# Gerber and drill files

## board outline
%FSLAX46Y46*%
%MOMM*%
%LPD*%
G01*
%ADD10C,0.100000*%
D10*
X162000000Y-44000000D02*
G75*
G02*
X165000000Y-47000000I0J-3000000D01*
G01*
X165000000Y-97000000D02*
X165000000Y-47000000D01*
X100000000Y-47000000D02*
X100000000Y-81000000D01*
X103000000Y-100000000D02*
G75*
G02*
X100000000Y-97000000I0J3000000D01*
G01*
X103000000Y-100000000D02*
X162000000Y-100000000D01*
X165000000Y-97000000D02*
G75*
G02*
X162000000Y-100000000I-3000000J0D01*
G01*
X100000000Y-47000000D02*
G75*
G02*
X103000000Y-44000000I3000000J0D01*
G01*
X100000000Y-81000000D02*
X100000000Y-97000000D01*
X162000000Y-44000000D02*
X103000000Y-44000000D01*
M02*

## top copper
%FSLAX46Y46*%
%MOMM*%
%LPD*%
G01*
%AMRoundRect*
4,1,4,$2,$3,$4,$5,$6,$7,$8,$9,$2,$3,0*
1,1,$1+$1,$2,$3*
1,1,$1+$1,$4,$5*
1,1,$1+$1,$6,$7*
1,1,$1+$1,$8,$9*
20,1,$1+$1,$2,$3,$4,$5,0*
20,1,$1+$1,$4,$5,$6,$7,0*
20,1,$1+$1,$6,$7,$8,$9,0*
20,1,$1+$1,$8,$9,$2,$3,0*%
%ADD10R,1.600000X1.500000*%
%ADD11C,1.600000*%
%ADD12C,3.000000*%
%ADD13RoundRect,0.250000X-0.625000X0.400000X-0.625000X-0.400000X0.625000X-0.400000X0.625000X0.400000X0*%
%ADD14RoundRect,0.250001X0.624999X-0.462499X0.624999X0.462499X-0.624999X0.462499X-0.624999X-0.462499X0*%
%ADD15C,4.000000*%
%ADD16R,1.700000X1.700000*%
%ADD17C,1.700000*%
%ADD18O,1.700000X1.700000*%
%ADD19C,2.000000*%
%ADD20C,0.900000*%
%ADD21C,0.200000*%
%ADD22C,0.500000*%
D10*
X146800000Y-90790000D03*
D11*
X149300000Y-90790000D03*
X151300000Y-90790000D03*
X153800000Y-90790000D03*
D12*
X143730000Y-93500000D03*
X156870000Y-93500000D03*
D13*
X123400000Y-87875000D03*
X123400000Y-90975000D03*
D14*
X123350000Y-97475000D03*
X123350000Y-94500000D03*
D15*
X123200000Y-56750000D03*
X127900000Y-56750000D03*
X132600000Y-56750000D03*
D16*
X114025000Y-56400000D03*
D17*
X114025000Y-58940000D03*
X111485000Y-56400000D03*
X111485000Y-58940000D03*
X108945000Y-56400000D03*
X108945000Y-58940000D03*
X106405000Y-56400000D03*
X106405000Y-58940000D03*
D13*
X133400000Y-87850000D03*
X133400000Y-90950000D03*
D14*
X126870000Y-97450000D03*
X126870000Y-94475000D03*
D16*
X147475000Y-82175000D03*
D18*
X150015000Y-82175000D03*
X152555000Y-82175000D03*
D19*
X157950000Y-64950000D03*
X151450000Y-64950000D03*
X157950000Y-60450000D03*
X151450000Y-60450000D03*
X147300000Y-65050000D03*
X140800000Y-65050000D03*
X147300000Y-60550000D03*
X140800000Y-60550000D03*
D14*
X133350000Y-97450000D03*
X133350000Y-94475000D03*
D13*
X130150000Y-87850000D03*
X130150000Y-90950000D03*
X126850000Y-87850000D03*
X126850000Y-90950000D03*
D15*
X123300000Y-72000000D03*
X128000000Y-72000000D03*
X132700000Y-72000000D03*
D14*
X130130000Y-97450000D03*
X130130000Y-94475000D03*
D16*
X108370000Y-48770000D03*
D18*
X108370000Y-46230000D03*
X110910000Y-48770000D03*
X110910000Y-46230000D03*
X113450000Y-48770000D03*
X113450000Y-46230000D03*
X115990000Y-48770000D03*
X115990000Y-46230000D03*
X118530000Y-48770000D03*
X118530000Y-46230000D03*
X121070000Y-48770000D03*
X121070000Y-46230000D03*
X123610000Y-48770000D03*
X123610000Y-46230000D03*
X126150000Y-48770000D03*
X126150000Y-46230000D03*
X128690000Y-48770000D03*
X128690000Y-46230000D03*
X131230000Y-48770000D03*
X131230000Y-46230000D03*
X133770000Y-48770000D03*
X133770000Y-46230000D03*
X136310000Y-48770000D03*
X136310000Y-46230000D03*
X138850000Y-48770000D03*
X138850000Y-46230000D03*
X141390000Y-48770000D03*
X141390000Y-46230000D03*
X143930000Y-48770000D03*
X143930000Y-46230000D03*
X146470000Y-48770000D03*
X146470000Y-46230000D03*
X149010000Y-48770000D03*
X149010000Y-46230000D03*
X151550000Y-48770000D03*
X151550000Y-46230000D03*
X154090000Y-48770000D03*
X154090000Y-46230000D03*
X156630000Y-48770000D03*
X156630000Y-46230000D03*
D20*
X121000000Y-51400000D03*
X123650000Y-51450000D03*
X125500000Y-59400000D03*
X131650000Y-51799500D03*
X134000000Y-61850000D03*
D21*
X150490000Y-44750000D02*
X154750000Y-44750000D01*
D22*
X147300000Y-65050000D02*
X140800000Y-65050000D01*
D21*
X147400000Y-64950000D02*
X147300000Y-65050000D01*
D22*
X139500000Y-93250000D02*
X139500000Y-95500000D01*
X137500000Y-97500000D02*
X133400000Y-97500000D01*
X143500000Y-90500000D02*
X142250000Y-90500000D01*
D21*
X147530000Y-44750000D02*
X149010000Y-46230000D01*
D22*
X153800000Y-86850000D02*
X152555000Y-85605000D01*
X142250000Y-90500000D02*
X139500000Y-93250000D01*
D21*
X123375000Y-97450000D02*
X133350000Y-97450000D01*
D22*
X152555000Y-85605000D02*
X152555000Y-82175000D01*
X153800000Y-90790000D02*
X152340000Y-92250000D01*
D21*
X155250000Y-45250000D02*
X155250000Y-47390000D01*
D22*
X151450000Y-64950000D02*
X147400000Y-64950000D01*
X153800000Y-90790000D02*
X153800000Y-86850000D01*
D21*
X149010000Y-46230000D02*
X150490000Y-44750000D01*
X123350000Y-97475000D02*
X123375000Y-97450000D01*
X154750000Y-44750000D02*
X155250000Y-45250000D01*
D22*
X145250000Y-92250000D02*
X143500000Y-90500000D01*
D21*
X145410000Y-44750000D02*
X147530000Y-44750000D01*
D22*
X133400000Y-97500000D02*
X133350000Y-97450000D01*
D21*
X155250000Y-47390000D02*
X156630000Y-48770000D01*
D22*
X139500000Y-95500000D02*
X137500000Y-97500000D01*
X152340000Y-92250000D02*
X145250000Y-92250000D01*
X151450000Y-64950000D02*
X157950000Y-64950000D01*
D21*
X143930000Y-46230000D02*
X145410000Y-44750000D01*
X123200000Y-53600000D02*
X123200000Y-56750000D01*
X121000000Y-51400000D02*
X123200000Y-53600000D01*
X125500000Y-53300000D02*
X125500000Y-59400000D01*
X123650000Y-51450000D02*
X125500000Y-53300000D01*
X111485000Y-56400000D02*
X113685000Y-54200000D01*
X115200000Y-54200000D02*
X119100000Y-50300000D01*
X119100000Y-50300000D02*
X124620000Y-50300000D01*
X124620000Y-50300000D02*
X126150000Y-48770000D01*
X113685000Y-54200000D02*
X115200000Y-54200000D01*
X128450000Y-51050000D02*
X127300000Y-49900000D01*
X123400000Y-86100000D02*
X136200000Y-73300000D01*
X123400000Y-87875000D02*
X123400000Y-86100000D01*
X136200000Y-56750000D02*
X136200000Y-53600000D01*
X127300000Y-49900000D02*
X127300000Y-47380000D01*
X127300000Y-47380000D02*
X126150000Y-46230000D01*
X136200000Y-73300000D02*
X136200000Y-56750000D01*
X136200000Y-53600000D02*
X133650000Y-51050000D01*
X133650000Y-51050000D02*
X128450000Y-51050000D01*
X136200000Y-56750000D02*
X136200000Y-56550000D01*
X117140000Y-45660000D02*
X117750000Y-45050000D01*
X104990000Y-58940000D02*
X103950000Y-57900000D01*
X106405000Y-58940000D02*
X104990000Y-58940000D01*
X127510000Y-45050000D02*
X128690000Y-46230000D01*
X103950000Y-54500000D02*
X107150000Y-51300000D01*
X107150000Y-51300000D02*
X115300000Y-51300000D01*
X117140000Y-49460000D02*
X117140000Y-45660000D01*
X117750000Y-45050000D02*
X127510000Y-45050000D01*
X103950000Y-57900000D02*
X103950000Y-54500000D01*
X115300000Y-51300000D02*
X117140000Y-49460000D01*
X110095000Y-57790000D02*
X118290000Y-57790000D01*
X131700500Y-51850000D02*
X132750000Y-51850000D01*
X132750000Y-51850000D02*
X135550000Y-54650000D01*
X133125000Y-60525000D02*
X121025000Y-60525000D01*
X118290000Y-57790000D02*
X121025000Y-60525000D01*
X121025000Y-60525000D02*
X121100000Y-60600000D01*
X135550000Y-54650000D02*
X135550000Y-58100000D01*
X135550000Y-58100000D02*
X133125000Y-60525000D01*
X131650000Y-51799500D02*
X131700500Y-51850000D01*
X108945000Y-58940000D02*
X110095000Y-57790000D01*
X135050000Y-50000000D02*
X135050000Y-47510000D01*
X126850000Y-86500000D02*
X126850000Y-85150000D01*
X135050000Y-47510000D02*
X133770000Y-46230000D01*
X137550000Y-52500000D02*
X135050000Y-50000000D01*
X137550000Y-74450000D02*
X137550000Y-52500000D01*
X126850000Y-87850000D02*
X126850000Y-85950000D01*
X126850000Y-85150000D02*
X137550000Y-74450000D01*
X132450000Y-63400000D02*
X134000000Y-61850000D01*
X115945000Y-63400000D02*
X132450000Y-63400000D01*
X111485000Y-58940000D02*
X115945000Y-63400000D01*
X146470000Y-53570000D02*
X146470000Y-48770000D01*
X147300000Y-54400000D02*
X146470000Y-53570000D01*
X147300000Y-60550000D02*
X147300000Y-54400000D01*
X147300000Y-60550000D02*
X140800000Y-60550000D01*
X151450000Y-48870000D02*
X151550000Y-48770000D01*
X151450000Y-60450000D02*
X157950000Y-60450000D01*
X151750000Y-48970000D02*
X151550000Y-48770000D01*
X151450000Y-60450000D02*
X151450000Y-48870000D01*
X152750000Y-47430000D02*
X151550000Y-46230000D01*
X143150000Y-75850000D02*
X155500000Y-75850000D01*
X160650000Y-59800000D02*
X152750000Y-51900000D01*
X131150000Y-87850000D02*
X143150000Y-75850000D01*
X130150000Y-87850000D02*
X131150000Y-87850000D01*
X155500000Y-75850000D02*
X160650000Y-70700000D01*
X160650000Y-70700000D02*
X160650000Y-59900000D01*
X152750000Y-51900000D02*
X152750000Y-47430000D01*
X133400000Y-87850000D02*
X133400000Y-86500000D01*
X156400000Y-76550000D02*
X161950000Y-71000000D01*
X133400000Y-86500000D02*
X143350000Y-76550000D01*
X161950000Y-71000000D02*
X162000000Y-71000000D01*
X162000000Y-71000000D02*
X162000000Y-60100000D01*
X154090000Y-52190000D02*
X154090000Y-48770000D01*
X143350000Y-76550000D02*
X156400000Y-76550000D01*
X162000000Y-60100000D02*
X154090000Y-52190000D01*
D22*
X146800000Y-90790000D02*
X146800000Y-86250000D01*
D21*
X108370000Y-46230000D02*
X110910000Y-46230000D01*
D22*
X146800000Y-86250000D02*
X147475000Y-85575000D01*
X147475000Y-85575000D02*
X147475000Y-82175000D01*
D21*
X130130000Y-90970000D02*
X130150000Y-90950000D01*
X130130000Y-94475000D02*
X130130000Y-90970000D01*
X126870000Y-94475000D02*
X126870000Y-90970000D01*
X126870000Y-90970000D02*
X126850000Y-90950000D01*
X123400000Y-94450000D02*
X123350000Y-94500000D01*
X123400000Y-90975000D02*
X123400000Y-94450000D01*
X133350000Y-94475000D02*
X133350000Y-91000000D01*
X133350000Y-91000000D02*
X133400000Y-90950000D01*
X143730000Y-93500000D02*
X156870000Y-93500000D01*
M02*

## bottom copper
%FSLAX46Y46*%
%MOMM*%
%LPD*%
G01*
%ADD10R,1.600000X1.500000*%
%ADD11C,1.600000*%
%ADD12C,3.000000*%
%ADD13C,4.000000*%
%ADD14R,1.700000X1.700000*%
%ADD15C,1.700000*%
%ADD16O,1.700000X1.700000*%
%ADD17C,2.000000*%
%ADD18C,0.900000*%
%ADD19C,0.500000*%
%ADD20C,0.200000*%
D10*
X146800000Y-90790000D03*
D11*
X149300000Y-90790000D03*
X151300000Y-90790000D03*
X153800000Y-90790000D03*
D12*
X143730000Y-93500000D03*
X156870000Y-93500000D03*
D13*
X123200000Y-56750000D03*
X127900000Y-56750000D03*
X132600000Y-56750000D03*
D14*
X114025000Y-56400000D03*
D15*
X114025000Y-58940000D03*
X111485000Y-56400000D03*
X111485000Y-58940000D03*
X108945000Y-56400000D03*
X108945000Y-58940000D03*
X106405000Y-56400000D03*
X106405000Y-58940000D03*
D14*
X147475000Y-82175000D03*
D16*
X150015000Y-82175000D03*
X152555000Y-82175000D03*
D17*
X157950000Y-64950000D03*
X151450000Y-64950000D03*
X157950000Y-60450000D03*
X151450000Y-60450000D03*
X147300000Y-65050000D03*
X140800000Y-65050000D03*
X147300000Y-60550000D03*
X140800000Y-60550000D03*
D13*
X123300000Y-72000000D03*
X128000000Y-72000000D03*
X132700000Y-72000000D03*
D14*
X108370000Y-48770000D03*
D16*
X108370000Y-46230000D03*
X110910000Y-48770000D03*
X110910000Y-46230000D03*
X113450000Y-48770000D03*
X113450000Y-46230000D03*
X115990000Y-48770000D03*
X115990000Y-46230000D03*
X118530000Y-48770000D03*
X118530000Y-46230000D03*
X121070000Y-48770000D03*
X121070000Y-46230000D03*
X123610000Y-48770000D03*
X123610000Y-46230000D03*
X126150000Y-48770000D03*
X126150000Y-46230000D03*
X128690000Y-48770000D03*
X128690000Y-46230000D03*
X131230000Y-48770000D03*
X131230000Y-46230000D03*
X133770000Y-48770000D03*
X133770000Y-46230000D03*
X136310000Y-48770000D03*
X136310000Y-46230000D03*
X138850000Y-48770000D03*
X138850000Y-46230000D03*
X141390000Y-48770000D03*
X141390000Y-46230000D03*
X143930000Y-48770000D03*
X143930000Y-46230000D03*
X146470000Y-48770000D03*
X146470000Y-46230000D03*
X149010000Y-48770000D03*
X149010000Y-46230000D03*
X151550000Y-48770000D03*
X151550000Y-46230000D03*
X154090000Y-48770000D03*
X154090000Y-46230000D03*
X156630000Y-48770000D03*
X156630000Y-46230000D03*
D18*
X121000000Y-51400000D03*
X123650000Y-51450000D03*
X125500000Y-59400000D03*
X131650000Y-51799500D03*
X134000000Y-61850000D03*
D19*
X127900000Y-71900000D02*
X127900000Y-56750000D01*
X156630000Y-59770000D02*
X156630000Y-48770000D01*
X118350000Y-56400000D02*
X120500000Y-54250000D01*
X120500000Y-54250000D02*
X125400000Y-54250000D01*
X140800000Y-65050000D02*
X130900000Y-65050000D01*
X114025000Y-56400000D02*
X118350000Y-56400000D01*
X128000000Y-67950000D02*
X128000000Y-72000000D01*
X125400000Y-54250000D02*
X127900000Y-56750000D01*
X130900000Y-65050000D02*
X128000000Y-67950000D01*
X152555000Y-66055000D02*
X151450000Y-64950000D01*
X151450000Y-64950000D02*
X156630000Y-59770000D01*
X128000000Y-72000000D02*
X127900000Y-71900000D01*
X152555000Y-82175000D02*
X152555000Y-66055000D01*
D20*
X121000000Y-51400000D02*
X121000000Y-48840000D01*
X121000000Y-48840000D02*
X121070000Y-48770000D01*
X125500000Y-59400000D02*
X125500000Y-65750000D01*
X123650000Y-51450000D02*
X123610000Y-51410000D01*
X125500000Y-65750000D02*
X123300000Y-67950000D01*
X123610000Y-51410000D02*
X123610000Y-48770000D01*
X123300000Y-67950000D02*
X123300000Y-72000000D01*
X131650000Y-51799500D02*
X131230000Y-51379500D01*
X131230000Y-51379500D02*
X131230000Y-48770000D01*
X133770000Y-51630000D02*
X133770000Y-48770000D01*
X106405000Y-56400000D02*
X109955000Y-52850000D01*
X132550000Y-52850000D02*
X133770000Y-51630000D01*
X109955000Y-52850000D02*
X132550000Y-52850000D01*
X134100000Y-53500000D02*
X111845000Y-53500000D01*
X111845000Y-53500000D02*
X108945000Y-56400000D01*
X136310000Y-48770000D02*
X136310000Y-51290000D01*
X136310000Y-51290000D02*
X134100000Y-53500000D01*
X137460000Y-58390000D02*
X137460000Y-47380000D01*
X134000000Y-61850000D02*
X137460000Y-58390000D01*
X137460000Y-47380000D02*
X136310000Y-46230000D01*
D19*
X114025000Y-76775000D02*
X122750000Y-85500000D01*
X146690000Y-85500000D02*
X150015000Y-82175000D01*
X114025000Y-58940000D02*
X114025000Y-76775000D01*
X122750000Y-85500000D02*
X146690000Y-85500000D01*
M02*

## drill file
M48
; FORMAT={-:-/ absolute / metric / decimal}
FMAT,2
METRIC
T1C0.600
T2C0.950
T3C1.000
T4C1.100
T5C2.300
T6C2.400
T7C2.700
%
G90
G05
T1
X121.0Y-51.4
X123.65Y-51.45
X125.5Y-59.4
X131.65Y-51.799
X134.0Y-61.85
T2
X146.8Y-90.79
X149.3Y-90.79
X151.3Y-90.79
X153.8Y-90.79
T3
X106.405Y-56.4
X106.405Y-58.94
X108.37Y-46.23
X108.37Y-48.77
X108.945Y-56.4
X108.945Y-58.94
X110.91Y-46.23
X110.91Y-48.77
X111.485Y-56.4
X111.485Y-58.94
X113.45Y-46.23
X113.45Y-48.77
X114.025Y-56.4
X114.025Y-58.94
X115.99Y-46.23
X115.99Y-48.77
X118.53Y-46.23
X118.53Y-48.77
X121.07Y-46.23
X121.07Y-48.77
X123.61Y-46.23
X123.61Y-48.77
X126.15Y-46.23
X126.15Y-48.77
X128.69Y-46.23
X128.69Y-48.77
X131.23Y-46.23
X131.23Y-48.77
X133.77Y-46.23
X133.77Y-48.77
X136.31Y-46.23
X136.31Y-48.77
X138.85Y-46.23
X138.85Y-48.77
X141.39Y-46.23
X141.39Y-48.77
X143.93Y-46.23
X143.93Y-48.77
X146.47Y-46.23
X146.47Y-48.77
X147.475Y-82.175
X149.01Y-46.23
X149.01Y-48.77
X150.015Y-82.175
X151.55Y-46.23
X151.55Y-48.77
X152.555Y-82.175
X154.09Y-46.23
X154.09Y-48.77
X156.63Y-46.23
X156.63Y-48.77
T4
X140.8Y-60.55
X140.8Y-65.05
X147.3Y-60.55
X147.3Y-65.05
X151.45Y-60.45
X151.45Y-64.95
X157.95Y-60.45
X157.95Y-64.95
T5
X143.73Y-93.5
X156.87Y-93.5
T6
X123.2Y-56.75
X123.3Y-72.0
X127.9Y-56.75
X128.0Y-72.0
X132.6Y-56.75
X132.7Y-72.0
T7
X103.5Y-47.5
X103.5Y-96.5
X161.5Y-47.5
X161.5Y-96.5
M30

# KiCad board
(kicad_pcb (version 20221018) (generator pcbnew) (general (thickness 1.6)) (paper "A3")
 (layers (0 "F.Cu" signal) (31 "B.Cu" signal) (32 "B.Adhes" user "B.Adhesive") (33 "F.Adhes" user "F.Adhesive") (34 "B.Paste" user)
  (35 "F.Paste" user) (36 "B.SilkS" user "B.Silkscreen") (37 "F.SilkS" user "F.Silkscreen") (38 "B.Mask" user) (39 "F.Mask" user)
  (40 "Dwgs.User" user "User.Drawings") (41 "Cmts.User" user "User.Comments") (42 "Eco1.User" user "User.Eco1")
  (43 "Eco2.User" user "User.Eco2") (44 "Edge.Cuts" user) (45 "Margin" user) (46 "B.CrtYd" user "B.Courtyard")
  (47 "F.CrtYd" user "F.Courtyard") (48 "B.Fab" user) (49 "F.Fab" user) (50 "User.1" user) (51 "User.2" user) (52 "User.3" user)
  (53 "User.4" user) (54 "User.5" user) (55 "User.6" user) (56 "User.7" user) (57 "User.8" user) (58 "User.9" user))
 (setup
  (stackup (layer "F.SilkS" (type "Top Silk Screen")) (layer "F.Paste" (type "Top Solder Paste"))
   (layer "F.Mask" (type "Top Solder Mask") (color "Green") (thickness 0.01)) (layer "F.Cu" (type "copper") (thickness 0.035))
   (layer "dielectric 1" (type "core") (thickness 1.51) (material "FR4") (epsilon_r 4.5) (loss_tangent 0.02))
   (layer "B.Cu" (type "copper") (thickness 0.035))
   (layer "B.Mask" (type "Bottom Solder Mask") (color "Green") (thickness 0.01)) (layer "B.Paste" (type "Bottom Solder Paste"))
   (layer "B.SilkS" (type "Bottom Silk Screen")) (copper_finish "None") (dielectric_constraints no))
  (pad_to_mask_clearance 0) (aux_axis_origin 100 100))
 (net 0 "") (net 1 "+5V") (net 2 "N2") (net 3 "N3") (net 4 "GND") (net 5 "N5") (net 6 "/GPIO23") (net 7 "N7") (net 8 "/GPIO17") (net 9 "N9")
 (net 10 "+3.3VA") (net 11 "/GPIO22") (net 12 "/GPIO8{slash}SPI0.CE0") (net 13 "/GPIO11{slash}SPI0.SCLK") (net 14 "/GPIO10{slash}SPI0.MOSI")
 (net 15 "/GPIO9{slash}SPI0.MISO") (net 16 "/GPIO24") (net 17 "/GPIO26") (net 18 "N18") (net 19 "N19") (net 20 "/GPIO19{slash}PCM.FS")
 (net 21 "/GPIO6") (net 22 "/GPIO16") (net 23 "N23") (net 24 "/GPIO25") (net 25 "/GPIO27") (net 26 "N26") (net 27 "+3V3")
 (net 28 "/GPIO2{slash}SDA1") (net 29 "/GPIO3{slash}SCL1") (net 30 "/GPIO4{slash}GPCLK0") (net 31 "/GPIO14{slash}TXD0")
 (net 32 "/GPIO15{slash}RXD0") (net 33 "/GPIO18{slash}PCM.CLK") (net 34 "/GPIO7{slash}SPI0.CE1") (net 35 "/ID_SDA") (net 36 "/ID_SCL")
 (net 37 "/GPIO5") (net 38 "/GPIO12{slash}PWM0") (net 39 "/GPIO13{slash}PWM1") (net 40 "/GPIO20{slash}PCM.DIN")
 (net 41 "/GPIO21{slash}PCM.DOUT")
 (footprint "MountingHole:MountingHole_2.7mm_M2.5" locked (layer "F.Cu") (at 161.5 47.5)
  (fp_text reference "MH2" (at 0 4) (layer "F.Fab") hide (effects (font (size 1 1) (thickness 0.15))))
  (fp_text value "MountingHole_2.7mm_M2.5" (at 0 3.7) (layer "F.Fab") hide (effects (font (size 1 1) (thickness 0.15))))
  (pad "" np_thru_hole circle locked (at 0 0) (size 2.7 2.7) (drill 2.7) (layers "*.Cu" "*.Mask")))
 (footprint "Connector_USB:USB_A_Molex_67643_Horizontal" (layer "F.Cu") (at 146.8 90.79)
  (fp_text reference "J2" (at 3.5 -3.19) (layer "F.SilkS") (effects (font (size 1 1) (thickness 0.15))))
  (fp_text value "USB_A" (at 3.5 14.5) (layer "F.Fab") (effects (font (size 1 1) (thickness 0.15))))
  (pad "1" thru_hole rect (at 0 0) (size 1.6 1.5) (drill 0.95) (layers "*.Cu" "*.Mask") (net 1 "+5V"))
  (pad "2" thru_hole circle (at 2.5 0) (size 1.6 1.6) (drill 0.95) (layers "*.Cu" "*.Mask") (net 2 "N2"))
  (pad "3" thru_hole circle (at 4.5 0) (size 1.6 1.6) (drill 0.95) (layers "*.Cu" "*.Mask") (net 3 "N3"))
  (pad "4" thru_hole circle (at 7 0) (size 1.6 1.6) (drill 0.95) (layers "*.Cu" "*.Mask") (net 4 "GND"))
  (pad "5" thru_hole circle (at -3.07 2.71) (size 3 3) (drill 2.3) (layers "*.Cu" "*.Mask") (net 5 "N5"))
  (pad "5" thru_hole circle (at 10.07 2.71) (size 3 3) (drill 2.3) (layers "*.Cu" "*.Mask") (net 5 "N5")))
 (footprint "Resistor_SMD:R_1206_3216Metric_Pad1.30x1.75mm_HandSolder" (layer "F.Cu") (at 123.4 89.425 -90)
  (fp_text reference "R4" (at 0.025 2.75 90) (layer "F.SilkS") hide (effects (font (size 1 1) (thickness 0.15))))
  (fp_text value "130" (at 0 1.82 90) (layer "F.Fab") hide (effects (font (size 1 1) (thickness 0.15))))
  (pad "1" smd roundrect (at -1.55 0 270) (size 1.3 1.75) (layers "F.Cu" "F.Paste" "F.Mask") (roundrect_rratio 0.1923076923)
   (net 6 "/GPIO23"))
  (pad "2" smd roundrect (at 1.55 0 270) (size 1.3 1.75) (layers "F.Cu" "F.Paste" "F.Mask") (roundrect_rratio 0.1923076923) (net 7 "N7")))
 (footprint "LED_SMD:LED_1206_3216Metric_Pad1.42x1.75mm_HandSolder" (layer "F.Cu") (at 123.35 95.9875 90)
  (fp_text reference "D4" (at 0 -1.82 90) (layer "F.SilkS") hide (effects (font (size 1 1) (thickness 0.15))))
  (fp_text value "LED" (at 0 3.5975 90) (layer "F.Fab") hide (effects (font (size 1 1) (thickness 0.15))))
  (pad "1" smd roundrect (at -1.4875 0 90) (size 1.425 1.75) (layers "F.Cu" "F.Paste" "F.Mask") (roundrect_rratio 0.1754392982)
   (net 4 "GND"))
  (pad "2" smd roundrect (at 1.4875 0 90) (size 1.425 1.75) (layers "F.Cu" "F.Paste" "F.Mask") (roundrect_rratio 0.1754392982) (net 7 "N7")))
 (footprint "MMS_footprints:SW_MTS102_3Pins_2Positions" (layer "F.Cu") (at 127.9 56.75)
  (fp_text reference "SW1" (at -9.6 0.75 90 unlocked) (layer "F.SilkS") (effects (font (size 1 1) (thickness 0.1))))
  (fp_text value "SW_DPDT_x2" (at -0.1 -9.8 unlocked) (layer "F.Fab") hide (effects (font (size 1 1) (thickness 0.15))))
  (pad "1" thru_hole circle (at -4.7 0) (size 4 4) (drill 2.4) (layers "*.Cu" "*.Mask") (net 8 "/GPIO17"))
  (pad "2" thru_hole circle (at 0 0) (size 4 4) (drill 2.4) (layers "*.Cu" "*.Mask") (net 4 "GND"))
  (pad "3" thru_hole circle (at 4.7 0) (size 4 4) (drill 2.4) (layers "*.Cu" "*.Mask") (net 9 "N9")))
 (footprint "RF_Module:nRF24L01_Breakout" (layer "F.Cu") (at 114.025 56.4 -90)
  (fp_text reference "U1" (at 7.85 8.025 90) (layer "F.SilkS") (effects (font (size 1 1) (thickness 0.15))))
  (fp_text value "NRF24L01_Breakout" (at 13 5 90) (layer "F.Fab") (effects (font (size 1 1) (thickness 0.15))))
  (pad "1" thru_hole rect (at 0 0 270) (size 1.7 1.7) (drill 1) (layers "*.Cu" "*.Mask") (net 4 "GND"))
  (pad "2" thru_hole circle (at 2.54 0 270) (size 1.7 1.7) (drill 1) (layers "*.Cu" "*.Mask") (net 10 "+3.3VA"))
  (pad "3" thru_hole circle (at 0 2.54 270) (size 1.7 1.7) (drill 1) (layers "*.Cu" "*.Mask") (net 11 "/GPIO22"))
  (pad "4" thru_hole circle (at 2.54 2.54 270) (size 1.7 1.7) (drill 1) (layers "*.Cu" "*.Mask") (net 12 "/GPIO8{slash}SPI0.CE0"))
  (pad "5" thru_hole circle (at 0 5.08 270) (size 1.7 1.7) (drill 1) (layers "*.Cu" "*.Mask") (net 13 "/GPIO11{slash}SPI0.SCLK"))
  (pad "6" thru_hole circle (at 2.54 5.08 270) (size 1.7 1.7) (drill 1) (layers "*.Cu" "*.Mask") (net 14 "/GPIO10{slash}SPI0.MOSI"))
  (pad "7" thru_hole circle (at 0 7.62 270) (size 1.7 1.7) (drill 1) (layers "*.Cu" "*.Mask") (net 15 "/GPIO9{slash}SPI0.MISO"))
  (pad "8" thru_hole circle (at 2.54 7.62 270) (size 1.7 1.7) (drill 1) (layers "*.Cu" "*.Mask") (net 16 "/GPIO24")))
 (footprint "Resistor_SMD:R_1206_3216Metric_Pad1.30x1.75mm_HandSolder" (layer "F.Cu") (at 133.4 89.4 -90)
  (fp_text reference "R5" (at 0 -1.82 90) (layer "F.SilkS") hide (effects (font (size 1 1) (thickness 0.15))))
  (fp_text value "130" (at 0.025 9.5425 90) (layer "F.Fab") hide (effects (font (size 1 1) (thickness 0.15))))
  (pad "1" smd roundrect (at -1.55 0 270) (size 1.3 1.75) (layers "F.Cu" "F.Paste" "F.Mask") (roundrect_rratio 0.1923076923)
   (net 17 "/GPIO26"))
  (pad "2" smd roundrect (at 1.55 0 270) (size 1.3 1.75) (layers "F.Cu" "F.Paste" "F.Mask") (roundrect_rratio 0.1923076923) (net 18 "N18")))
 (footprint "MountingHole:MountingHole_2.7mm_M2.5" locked (layer "F.Cu") (at 103.5 96.5)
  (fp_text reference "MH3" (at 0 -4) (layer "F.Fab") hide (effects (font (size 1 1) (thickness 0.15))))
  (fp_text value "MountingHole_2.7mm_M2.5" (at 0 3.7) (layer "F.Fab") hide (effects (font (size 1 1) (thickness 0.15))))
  (pad "" np_thru_hole circle locked (at 0 0) (size 2.7 2.7) (drill 2.7) (layers "*.Cu" "*.Mask")))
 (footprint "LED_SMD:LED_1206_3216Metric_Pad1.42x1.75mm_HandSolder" (layer "F.Cu") (at 126.87 95.9625 90)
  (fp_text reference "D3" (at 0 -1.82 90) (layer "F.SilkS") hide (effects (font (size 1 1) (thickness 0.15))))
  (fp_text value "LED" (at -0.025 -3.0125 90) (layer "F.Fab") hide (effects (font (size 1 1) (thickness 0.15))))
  (pad "1" smd roundrect (at -1.4875 0 90) (size 1.425 1.75) (layers "F.Cu" "F.Paste" "F.Mask") (roundrect_rratio 0.1754392982)
   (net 4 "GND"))
  (pad "2" smd roundrect (at 1.4875 0 90) (size 1.425 1.75) (layers "F.Cu" "F.Paste" "F.Mask") (roundrect_rratio 0.1754392982)
   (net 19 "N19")))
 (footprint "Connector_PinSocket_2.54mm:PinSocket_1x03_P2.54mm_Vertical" (layer "F.Cu") (at 147.475 82.175 90)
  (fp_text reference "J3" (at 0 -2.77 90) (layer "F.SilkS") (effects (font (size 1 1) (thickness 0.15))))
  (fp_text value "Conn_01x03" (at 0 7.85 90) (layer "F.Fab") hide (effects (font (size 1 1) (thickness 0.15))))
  (pad "1" thru_hole rect (at 0 0 90) (size 1.7 1.7) (drill 1) (layers "*.Cu" "*.Mask") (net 1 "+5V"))
  (pad "2" thru_hole oval (at 0 2.54 90) (size 1.7 1.7) (drill 1) (layers "*.Cu" "*.Mask") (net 10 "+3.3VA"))
  (pad "3" thru_hole oval (at 0 5.08 90) (size 1.7 1.7) (drill 1) (layers "*.Cu" "*.Mask") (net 4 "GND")))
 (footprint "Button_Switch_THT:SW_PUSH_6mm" (layer "F.Cu") (at 157.95 64.95 180)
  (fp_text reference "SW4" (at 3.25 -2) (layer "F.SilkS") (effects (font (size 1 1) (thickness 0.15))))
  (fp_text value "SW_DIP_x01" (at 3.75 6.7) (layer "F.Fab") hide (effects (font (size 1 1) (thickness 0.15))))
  (pad "1" thru_hole circle (at 0 0 270) (size 2 2) (drill 1.1) (layers "*.Cu" "*.Mask") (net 4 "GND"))
  (pad "1" thru_hole circle (at 6.5 0 270) (size 2 2) (drill 1.1) (layers "*.Cu" "*.Mask") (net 4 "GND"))
  (pad "2" thru_hole circle (at 0 4.5 270) (size 2 2) (drill 1.1) (layers "*.Cu" "*.Mask") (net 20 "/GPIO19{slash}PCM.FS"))
  (pad "2" thru_hole circle (at 6.5 4.5 270) (size 2 2) (drill 1.1) (layers "*.Cu" "*.Mask") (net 20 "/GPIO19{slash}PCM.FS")))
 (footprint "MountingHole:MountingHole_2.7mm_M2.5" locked (layer "F.Cu") (at 103.5 47.5)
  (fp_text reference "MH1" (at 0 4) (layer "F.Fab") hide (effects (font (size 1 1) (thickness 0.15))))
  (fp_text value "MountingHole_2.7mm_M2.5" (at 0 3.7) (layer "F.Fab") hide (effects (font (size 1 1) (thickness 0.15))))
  (pad "" np_thru_hole circle locked (at 0 0) (size 2.7 2.7) (drill 2.7) (layers "*.Cu" "*.Mask")))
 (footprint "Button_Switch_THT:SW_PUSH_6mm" (layer "F.Cu") (at 147.3 65.05 180)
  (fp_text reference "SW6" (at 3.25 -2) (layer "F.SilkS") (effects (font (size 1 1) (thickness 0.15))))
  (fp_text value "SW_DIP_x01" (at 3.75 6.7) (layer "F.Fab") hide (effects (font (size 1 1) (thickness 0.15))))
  (pad "1" thru_hole circle (at 0 0 270) (size 2 2) (drill 1.1) (layers "*.Cu" "*.Mask") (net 4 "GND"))
  (pad "1" thru_hole circle (at 6.5 0 270) (size 2 2) (drill 1.1) (layers "*.Cu" "*.Mask") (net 4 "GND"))
  (pad "2" thru_hole circle (at 0 4.5 270) (size 2 2) (drill 1.1) (layers "*.Cu" "*.Mask") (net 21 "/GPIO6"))
  (pad "2" thru_hole circle (at 6.5 4.5 270) (size 2 2) (drill 1.1) (layers "*.Cu" "*.Mask") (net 21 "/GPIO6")))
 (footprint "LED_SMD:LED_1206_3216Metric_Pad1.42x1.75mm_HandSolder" (layer "F.Cu") (at 133.35 95.9625 90)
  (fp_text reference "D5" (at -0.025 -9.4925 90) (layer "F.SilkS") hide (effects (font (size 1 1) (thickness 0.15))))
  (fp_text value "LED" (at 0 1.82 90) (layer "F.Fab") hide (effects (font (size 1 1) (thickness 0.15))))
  (pad "1" smd roundrect (at -1.4875 0 90) (size 1.425 1.75) (layers "F.Cu" "F.Paste" "F.Mask") (roundrect_rratio 0.1754392982)
   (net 4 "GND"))
  (pad "2" smd roundrect (at 1.4875 0 90) (size 1.425 1.75) (layers "F.Cu" "F.Paste" "F.Mask") (roundrect_rratio 0.1754392982)
   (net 18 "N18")))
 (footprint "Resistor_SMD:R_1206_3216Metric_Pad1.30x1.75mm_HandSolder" (layer "F.Cu") (at 130.15 89.4 -90)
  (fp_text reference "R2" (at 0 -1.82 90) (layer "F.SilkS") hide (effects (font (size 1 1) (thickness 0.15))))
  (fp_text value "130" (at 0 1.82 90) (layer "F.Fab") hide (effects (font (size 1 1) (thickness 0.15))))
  (pad "1" smd roundrect (at -1.55 0 270) (size 1.3 1.75) (layers "F.Cu" "F.Paste" "F.Mask") (roundrect_rratio 0.1923076923)
   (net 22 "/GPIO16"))
  (pad "2" smd roundrect (at 1.55 0 270) (size 1.3 1.75) (layers "F.Cu" "F.Paste" "F.Mask") (roundrect_rratio 0.1923076923) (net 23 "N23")))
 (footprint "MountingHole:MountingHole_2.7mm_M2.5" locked (layer "F.Cu") (at 161.5 96.5)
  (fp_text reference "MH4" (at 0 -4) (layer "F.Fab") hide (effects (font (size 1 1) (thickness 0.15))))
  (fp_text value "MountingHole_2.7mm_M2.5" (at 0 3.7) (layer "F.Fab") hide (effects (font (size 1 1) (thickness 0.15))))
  (pad "" np_thru_hole circle locked (at 0 0) (size 2.7 2.7) (drill 2.7) (layers "*.Cu" "*.Mask")))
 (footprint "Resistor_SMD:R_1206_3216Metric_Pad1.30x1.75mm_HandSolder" (layer "F.Cu") (at 126.85 89.4 -90)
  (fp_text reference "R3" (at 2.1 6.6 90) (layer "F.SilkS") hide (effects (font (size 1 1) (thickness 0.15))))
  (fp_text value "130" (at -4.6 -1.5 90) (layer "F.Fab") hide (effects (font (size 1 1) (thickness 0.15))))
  (pad "1" smd roundrect (at -1.55 0 270) (size 1.3 1.75) (layers "F.Cu" "F.Paste" "F.Mask") (roundrect_rratio 0.1923076923)
   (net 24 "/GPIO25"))
  (pad "2" smd roundrect (at 1.55 0 270) (size 1.3 1.75) (layers "F.Cu" "F.Paste" "F.Mask") (roundrect_rratio 0.1923076923) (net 19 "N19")))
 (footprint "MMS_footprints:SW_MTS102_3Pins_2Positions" (layer "F.Cu") (at 128 72)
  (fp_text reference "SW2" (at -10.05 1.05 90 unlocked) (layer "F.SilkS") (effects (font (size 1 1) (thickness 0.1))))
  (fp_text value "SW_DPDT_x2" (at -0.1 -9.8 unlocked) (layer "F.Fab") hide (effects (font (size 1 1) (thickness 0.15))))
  (pad "1" thru_hole circle (at -4.7 0) (size 4 4) (drill 2.4) (layers "*.Cu" "*.Mask") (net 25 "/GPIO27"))
  (pad "2" thru_hole circle (at 0 0) (size 4 4) (drill 2.4) (layers "*.Cu" "*.Mask") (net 4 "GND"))
  (pad "3" thru_hole circle (at 4.7 0) (size 4 4) (drill 2.4) (layers "*.Cu" "*.Mask") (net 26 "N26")))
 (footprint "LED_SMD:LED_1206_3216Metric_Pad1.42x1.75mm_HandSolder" (layer "F.Cu") (at 130.13 95.9625 90)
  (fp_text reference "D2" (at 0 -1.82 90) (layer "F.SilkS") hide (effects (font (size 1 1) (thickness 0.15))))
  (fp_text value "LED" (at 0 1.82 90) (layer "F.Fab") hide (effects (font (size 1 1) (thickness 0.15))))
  (pad "1" smd roundrect (at -1.4875 0 90) (size 1.425 1.75) (layers "F.Cu" "F.Paste" "F.Mask") (roundrect_rratio 0.1754392982)
   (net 4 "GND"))
  (pad "2" smd roundrect (at 1.4875 0 90) (size 1.425 1.75) (layers "F.Cu" "F.Paste" "F.Mask") (roundrect_rratio 0.1754392982)
   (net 23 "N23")))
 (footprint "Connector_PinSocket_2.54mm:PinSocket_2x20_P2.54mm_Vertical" (layer "B.Cu") (at 108.37 48.77 -90)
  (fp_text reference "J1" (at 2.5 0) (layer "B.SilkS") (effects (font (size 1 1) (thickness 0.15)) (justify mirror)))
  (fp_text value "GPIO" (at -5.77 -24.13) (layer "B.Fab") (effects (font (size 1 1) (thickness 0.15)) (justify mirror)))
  (pad "1" thru_hole rect (at 0 0 270) (size 1.7 1.7) (drill 1) (layers "*.Cu" "*.Mask") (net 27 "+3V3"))
  (pad "2" thru_hole oval (at -2.54 0 270) (size 1.7 1.7) (drill 1) (layers "*.Cu" "*.Mask") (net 1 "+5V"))
  (pad "3" thru_hole oval (at 0 -2.54 270) (size 1.7 1.7) (drill 1) (layers "*.Cu" "*.Mask") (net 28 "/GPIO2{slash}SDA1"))
  (pad "4" thru_hole oval (at -2.54 -2.54 270) (size 1.7 1.7) (drill 1) (layers "*.Cu" "*.Mask") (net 1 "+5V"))
  (pad "5" thru_hole oval (at 0 -5.08 270) (size 1.7 1.7) (drill 1) (layers "*.Cu" "*.Mask") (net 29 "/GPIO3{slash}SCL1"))
  (pad "6" thru_hole oval (at -2.54 -5.08 270) (size 1.7 1.7) (drill 1) (layers "*.Cu" "*.Mask") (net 4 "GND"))
  (pad "7" thru_hole oval (at 0 -7.62 270) (size 1.7 1.7) (drill 1) (layers "*.Cu" "*.Mask") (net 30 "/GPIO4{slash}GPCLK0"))
  (pad "8" thru_hole oval (at -2.54 -7.62 270) (size 1.7 1.7) (drill 1) (layers "*.Cu" "*.Mask") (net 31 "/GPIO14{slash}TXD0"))
  (pad "9" thru_hole oval (at 0 -10.16 270) (size 1.7 1.7) (drill 1) (layers "*.Cu" "*.Mask") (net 4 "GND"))
  (pad "10" thru_hole oval (at -2.54 -10.16 270) (size 1.7 1.7) (drill 1) (layers "*.Cu" "*.Mask") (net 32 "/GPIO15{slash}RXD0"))
  (pad "11" thru_hole oval (at 0 -12.7 270) (size 1.7 1.7) (drill 1) (layers "*.Cu" "*.Mask") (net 8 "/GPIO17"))
  (pad "12" thru_hole oval (at -2.54 -12.7 270) (size 1.7 1.7) (drill 1) (layers "*.Cu" "*.Mask") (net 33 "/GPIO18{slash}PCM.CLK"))
  (pad "13" thru_hole oval (at 0 -15.24 270) (size 1.7 1.7) (drill 1) (layers "*.Cu" "*.Mask") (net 25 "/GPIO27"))
  (pad "14" thru_hole oval (at -2.54 -15.24 270) (size 1.7 1.7) (drill 1) (layers "*.Cu" "*.Mask") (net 4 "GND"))
  (pad "15" thru_hole oval (at 0 -17.78 270) (size 1.7 1.7) (drill 1) (layers "*.Cu" "*.Mask") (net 11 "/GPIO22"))
  (pad "16" thru_hole oval (at -2.54 -17.78 270) (size 1.7 1.7) (drill 1) (layers "*.Cu" "*.Mask") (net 6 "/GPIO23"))
  (pad "17" thru_hole oval (at 0 -20.32 270) (size 1.7 1.7) (drill 1) (layers "*.Cu" "*.Mask") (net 27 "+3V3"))
  (pad "18" thru_hole oval (at -2.54 -20.32 270) (size 1.7 1.7) (drill 1) (layers "*.Cu" "*.Mask") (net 16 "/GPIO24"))
  (pad "19" thru_hole oval (at 0 -22.86 270) (size 1.7 1.7) (drill 1) (layers "*.Cu" "*.Mask") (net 14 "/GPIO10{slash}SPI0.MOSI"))
  (pad "20" thru_hole oval (at -2.54 -22.86 270) (size 1.7 1.7) (drill 1) (layers "*.Cu" "*.Mask") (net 4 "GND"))
  (pad "21" thru_hole oval (at 0 -25.4 270) (size 1.7 1.7) (drill 1) (layers "*.Cu" "*.Mask") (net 15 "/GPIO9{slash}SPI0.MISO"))
  (pad "22" thru_hole oval (at -2.54 -25.4 270) (size 1.7 1.7) (drill 1) (layers "*.Cu" "*.Mask") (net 24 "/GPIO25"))
  (pad "23" thru_hole oval (at 0 -27.94 270) (size 1.7 1.7) (drill 1) (layers "*.Cu" "*.Mask") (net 13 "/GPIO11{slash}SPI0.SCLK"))
  (pad "24" thru_hole oval (at -2.54 -27.94 270) (size 1.7 1.7) (drill 1) (layers "*.Cu" "*.Mask") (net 12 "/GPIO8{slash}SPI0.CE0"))
  (pad "25" thru_hole oval (at 0 -30.48 270) (size 1.7 1.7) (drill 1) (layers "*.Cu" "*.Mask") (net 4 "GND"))
  (pad "26" thru_hole oval (at -2.54 -30.48 270) (size 1.7 1.7) (drill 1) (layers "*.Cu" "*.Mask") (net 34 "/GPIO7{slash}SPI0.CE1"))
  (pad "27" thru_hole oval (at 0 -33.02 270) (size 1.7 1.7) (drill 1) (layers "*.Cu" "*.Mask") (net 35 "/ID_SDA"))
  (pad "28" thru_hole oval (at -2.54 -33.02 270) (size 1.7 1.7) (drill 1) (layers "*.Cu" "*.Mask") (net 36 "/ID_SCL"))
  (pad "29" thru_hole oval (at 0 -35.56 270) (size 1.7 1.7) (drill 1) (layers "*.Cu" "*.Mask") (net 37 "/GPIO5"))
  (pad "30" thru_hole oval (at -2.54 -35.56 270) (size 1.7 1.7) (drill 1) (layers "*.Cu" "*.Mask") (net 4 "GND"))
  (pad "31" thru_hole oval (at 0 -38.1 270) (size 1.7 1.7) (drill 1) (layers "*.Cu" "*.Mask") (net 21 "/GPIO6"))
  (pad "32" thru_hole oval (at -2.54 -38.1 270) (size 1.7 1.7) (drill 1) (layers "*.Cu" "*.Mask") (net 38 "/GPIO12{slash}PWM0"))
  (pad "33" thru_hole oval (at 0 -40.64 270) (size 1.7 1.7) (drill 1) (layers "*.Cu" "*.Mask") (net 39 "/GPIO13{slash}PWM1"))
  (pad "34" thru_hole oval (at -2.54 -40.64 270) (size 1.7 1.7) (drill 1) (layers "*.Cu" "*.Mask") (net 4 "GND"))
  (pad "35" thru_hole oval (at 0 -43.18 270) (size 1.7 1.7) (drill 1) (layers "*.Cu" "*.Mask") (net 20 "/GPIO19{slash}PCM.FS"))
  (pad "36" thru_hole oval (at -2.54 -43.18 270) (size 1.7 1.7) (drill 1) (layers "*.Cu" "*.Mask") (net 22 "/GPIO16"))
  (pad "37" thru_hole oval (at 0 -45.72 270) (size 1.7 1.7) (drill 1) (layers "*.Cu" "*.Mask") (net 17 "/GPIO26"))
  (pad "38" thru_hole oval (at -2.54 -45.72 270) (size 1.7 1.7) (drill 1) (layers "*.Cu" "*.Mask") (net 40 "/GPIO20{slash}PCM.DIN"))
  (pad "39" thru_hole oval (at 0 -48.26 270) (size 1.7 1.7) (drill 1) (layers "*.Cu" "*.Mask") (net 4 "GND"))
  (pad "40" thru_hole oval (at -2.54 -48.26 270) (size 1.7 1.7) (drill 1) (layers "*.Cu" "*.Mask") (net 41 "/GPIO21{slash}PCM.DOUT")))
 (gr_arc (start 162 44) (mid 164.12132 44.87868) (end 165 47) (stroke (width 0.1) (type solid)) (layer "Edge.Cuts"))
 (gr_line (start 165 97) (end 165 47) (stroke (width 0.1) (type solid)) (layer "Edge.Cuts"))
 (gr_line (start 100 47) (end 100 81) (stroke (width 0.1) (type solid)) (layer "Edge.Cuts"))
 (gr_arc (start 103 100) (mid 100.87868 99.12132) (end 100 97) (stroke (width 0.1) (type solid)) (layer "Edge.Cuts"))
 (gr_line (start 103 100) (end 162 100) (stroke (width 0.1) (type solid)) (layer "Edge.Cuts"))
 (gr_arc (start 165 97) (mid 164.12132 99.12132) (end 162 100) (stroke (width 0.1) (type solid)) (layer "Edge.Cuts"))
 (gr_arc (start 100 47) (mid 100.87868 44.87868) (end 103 44) (stroke (width 0.1) (type solid)) (layer "Edge.Cuts"))
 (gr_line (start 100 81) (end 100 97) (stroke (width 0.1) (type solid)) (layer "Edge.Cuts"))
 (gr_line (start 162 44) (end 103 44) (stroke (width 0.1) (type solid)) (layer "Edge.Cuts"))
 (segment (start 150.49 44.75) (end 154.75 44.75) (width 0.2) (layer "F.Cu") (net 4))
 (segment (start 147.3 65.05) (end 140.8 65.05) (width 0.5) (layer "F.Cu") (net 4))
 (segment (start 147.4 64.95) (end 147.3 65.05) (width 0.2) (layer "F.Cu") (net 4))
 (segment (start 139.5 93.25) (end 139.5 95.5) (width 0.5) (layer "F.Cu") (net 4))
 (segment (start 137.5 97.5) (end 133.4 97.5) (width 0.5) (layer "F.Cu") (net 4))
 (segment (start 143.5 90.5) (end 142.25 90.5) (width 0.5) (layer "F.Cu") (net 4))
 (segment (start 147.53 44.75) (end 149.01 46.23) (width 0.2) (layer "F.Cu") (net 4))
 (segment (start 153.8 86.85) (end 152.555 85.605) (width 0.5) (layer "F.Cu") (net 4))
 (segment (start 142.25 90.5) (end 139.5 93.25) (width 0.5) (layer "F.Cu") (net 4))
 (segment (start 123.375 97.45) (end 133.35 97.45) (width 0.2) (layer "F.Cu") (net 4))
 (segment (start 152.555 85.605) (end 152.555 82.175) (width 0.5) (layer "F.Cu") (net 4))
 (segment (start 153.8 90.79) (end 152.34 92.25) (width 0.5) (layer "F.Cu") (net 4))
 (segment (start 155.25 45.25) (end 155.25 47.39) (width 0.2) (layer "F.Cu") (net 4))
 (segment (start 151.45 64.95) (end 147.4 64.95) (width 0.5) (layer "F.Cu") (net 4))
 (segment (start 153.8 90.79) (end 153.8 86.85) (width 0.5) (layer "F.Cu") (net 4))
 (segment (start 149.01 46.23) (end 150.49 44.75) (width 0.2) (layer "F.Cu") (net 4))
 (segment (start 123.35 97.475) (end 123.375 97.45) (width 0.2) (layer "F.Cu") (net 4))
 (segment (start 154.75 44.75) (end 155.25 45.25) (width 0.2) (layer "F.Cu") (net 4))
 (segment (start 145.25 92.25) (end 143.5 90.5) (width 0.5) (layer "F.Cu") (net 4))
 (segment (start 145.41 44.75) (end 147.53 44.75) (width 0.2) (layer "F.Cu") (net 4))
 (segment (start 133.4 97.5) (end 133.35 97.45) (width 0.5) (layer "F.Cu") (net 4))
 (segment (start 155.25 47.39) (end 156.63 48.77) (width 0.2) (layer "F.Cu") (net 4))
 (segment (start 139.5 95.5) (end 137.5 97.5) (width 0.5) (layer "F.Cu") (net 4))
 (segment (start 152.34 92.25) (end 145.25 92.25) (width 0.5) (layer "F.Cu") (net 4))
 (segment (start 151.45 64.95) (end 157.95 64.95) (width 0.5) (layer "F.Cu") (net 4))
 (segment (start 143.93 46.23) (end 145.41 44.75) (width 0.2) (layer "F.Cu") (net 4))
 (segment (start 127.9 71.9) (end 127.9 56.75) (width 0.5) (layer "B.Cu") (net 4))
 (segment (start 156.63 59.77) (end 156.63 48.77) (width 0.5) (layer "B.Cu") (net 4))
 (segment (start 118.35 56.4) (end 120.5 54.25) (width 0.5) (layer "B.Cu") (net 4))
 (segment (start 120.5 54.25) (end 125.4 54.25) (width 0.5) (layer "B.Cu") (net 4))
 (segment (start 140.8 65.05) (end 130.9 65.05) (width 0.5) (layer "B.Cu") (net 4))
 (segment (start 114.025 56.4) (end 118.35 56.4) (width 0.5) (layer "B.Cu") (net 4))
 (segment (start 128 67.95) (end 128 72) (width 0.5) (layer "B.Cu") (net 4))
 (segment (start 125.4 54.25) (end 127.9 56.75) (width 0.5) (layer "B.Cu") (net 4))
 (segment (start 130.9 65.05) (end 128 67.95) (width 0.5) (layer "B.Cu") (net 4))
 (segment (start 152.555 66.055) (end 151.45 64.95) (width 0.5) (layer "B.Cu") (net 4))
 (segment (start 151.45 64.95) (end 156.63 59.77) (width 0.5) (layer "B.Cu") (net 4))
 (segment (start 128 72) (end 127.9 71.9) (width 0.5) (layer "B.Cu") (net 4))
 (segment (start 152.555 82.175) (end 152.555 66.055) (width 0.5) (layer "B.Cu") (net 4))
 (segment (start 123.2 53.6) (end 123.2 56.75) (width 0.2) (layer "F.Cu") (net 8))
 (segment (start 121 51.4) (end 123.2 53.6) (width 0.2) (layer "F.Cu") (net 8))
 (via (at 121 51.4) (size 0.9) (drill 0.6) (layers "F.Cu" "B.Cu") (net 8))
 (segment (start 121 51.4) (end 121 48.84) (width 0.2) (layer "B.Cu") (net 8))
 (segment (start 121 48.84) (end 121.07 48.77) (width 0.2) (layer "B.Cu") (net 8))
 (segment (start 125.5 53.3) (end 125.5 59.4) (width 0.2) (layer "F.Cu") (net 25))
 (segment (start 123.65 51.45) (end 125.5 53.3) (width 0.2) (layer "F.Cu") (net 25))
 (via (at 123.65 51.45) (size 0.9) (drill 0.6) (layers "F.Cu" "B.Cu") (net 25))
 (via (at 125.5 59.4) (size 0.9) (drill 0.6) (layers "F.Cu" "B.Cu") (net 25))
 (segment (start 125.5 59.4) (end 125.5 65.75) (width 0.2) (layer "B.Cu") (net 25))
 (segment (start 123.65 51.45) (end 123.61 51.41) (width 0.2) (layer "B.Cu") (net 25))
 (segment (start 125.5 65.75) (end 123.3 67.95) (width 0.2) (layer "B.Cu") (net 25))
 (segment (start 123.61 51.41) (end 123.61 48.77) (width 0.2) (layer "B.Cu") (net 25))
 (segment (start 123.3 67.95) (end 123.3 72) (width 0.2) (layer "B.Cu") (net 25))
 (segment (start 111.485 56.4) (end 113.685 54.2) (width 0.2) (layer "F.Cu") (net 11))
 (segment (start 115.2 54.2) (end 119.1 50.3) (width 0.2) (layer "F.Cu") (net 11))
 (segment (start 119.1 50.3) (end 124.62 50.3) (width 0.2) (layer "F.Cu") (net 11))
 (segment (start 124.62 50.3) (end 126.15 48.77) (width 0.2) (layer "F.Cu") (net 11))
 (segment (start 113.685 54.2) (end 115.2 54.2) (width 0.2) (layer "F.Cu") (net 11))
 (segment (start 128.45 51.05) (end 127.3 49.9) (width 0.2) (layer "F.Cu") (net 6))
 (segment (start 123.4 86.1) (end 136.2 73.3) (width 0.2) (layer "F.Cu") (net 6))
 (segment (start 123.4 87.875) (end 123.4 86.1) (width 0.2) (layer "F.Cu") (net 6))
 (segment (start 136.2 56.75) (end 136.2 53.6) (width 0.2) (layer "F.Cu") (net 6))
 (segment (start 127.3 49.9) (end 127.3 47.38) (width 0.2) (layer "F.Cu") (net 6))
 (segment (start 127.3 47.38) (end 126.15 46.23) (width 0.2) (layer "F.Cu") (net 6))
 (segment (start 136.2 73.3) (end 136.2 56.75) (width 0.2) (layer "F.Cu") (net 6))
 (segment (start 136.2 53.6) (end 133.65 51.05) (width 0.2) (layer "F.Cu") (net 6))
 (segment (start 133.65 51.05) (end 128.45 51.05) (width 0.2) (layer "F.Cu") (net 6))
 (segment (start 136.2 56.75) (end 136.2 56.55) (width 0.2) (layer "F.Cu") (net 6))
 (segment (start 117.14 45.66) (end 117.75 45.05) (width 0.2) (layer "F.Cu") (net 16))
 (segment (start 104.99 58.94) (end 103.95 57.9) (width 0.2) (layer "F.Cu") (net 16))
 (segment (start 106.405 58.94) (end 104.99 58.94) (width 0.2) (layer "F.Cu") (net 16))
 (segment (start 127.51 45.05) (end 128.69 46.23) (width 0.2) (layer "F.Cu") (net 16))
 (segment (start 103.95 54.5) (end 107.15 51.3) (width 0.2) (layer "F.Cu") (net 16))
 (segment (start 107.15 51.3) (end 115.3 51.3) (width 0.2) (layer "F.Cu") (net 16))
 (segment (start 117.14 49.46) (end 117.14 45.66) (width 0.2) (layer "F.Cu") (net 16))
 (segment (start 117.75 45.05) (end 127.51 45.05) (width 0.2) (layer "F.Cu") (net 16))
 (segment (start 103.95 57.9) (end 103.95 54.5) (width 0.2) (layer "F.Cu") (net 16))
 (segment (start 115.3 51.3) (end 117.14 49.46) (width 0.2) (layer "F.Cu") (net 16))
 (segment (start 110.095 57.79) (end 118.29 57.79) (width 0.2) (layer "F.Cu") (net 14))
 (segment (start 131.7005 51.85) (end 132.75 51.85) (width 0.2) (layer "F.Cu") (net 14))
 (segment (start 132.75 51.85) (end 135.55 54.65) (width 0.2) (layer "F.Cu") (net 14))
 (segment (start 133.125 60.525) (end 121.025 60.525) (width 0.2) (layer "F.Cu") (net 14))
 (segment (start 118.29 57.79) (end 121.025 60.525) (width 0.2) (layer "F.Cu") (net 14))
 (segment (start 121.025 60.525) (end 121.1 60.6) (width 0.2) (layer "F.Cu") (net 14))
 (segment (start 135.55 54.65) (end 135.55 58.1) (width 0.2) (layer "F.Cu") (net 14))
 (segment (start 135.55 58.1) (end 133.125 60.525) (width 0.2) (layer "F.Cu") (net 14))
 (segment (start 131.65 51.7995) (end 131.7005 51.85) (width 0.2) (layer "F.Cu") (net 14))
 (segment (start 108.945 58.94) (end 110.095 57.79) (width 0.2) (layer "F.Cu") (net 14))
 (via (at 131.65 51.7995) (size 0.9) (drill 0.6) (layers "F.Cu" "B.Cu") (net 14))
 (segment (start 131.65 51.7995) (end 131.23 51.3795) (width 0.2) (layer "B.Cu") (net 14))
 (segment (start 131.23 51.3795) (end 131.23 48.77) (width 0.2) (layer "B.Cu") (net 14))
 (segment (start 133.77 51.63) (end 133.77 48.77) (width 0.2) (layer "B.Cu") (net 15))
 (segment (start 106.405 56.4) (end 109.955 52.85) (width 0.2) (layer "B.Cu") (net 15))
 (segment (start 132.55 52.85) (end 133.77 51.63) (width 0.2) (layer "B.Cu") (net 15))
 (segment (start 109.955 52.85) (end 132.55 52.85) (width 0.2) (layer "B.Cu") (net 15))
 (segment (start 135.05 50) (end 135.05 47.51) (width 0.2) (layer "F.Cu") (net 24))
 (segment (start 126.85 86.5) (end 126.85 85.15) (width 0.2) (layer "F.Cu") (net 24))
 (segment (start 135.05 47.51) (end 133.77 46.23) (width 0.2) (layer "F.Cu") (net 24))
 (segment (start 137.55 52.5) (end 135.05 50) (width 0.2) (layer "F.Cu") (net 24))
 (segment (start 137.55 74.45) (end 137.55 52.5) (width 0.2) (layer "F.Cu") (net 24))
 (segment (start 126.85 87.85) (end 126.85 85.95) (width 0.2) (layer "F.Cu") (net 24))
 (segment (start 126.85 85.15) (end 137.55 74.45) (width 0.2) (layer "F.Cu") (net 24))
 (segment (start 134.1 53.5) (end 111.845 53.5) (width 0.2) (layer "B.Cu") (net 13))
 (segment (start 111.845 53.5) (end 108.945 56.4) (width 0.2) (layer "B.Cu") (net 13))
 (segment (start 136.31 48.77) (end 136.31 51.29) (width 0.2) (layer "B.Cu") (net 13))
 (segment (start 136.31 51.29) (end 134.1 53.5) (width 0.2) (layer "B.Cu") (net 13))
 (segment (start 132.45 63.4) (end 134 61.85) (width 0.2) (layer "F.Cu") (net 12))
 (segment (start 115.945 63.4) (end 132.45 63.4) (width 0.2) (layer "F.Cu") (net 12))
 (segment (start 111.485 58.94) (end 115.945 63.4) (width 0.2) (layer "F.Cu") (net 12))
 (via (at 134 61.85) (size 0.9) (drill 0.6) (layers "F.Cu" "B.Cu") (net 12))
 (segment (start 137.46 58.39) (end 137.46 47.38) (width 0.2) (layer "B.Cu") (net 12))
 (segment (start 134 61.85) (end 137.46 58.39) (width 0.2) (layer "B.Cu") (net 12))
 (segment (start 137.46 47.38) (end 136.31 46.23) (width 0.2) (layer "B.Cu") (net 12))
 (segment (start 146.47 53.57) (end 146.47 48.77) (width 0.2) (layer "F.Cu") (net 21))
 (segment (start 147.3 54.4) (end 146.47 53.57) (width 0.2) (layer "F.Cu") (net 21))
 (segment (start 147.3 60.55) (end 147.3 54.4) (width 0.2) (layer "F.Cu") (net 21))
 (segment (start 147.3 60.55) (end 140.8 60.55) (width 0.2) (layer "F.Cu") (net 21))
 (segment (start 151.45 48.87) (end 151.55 48.77) (width 0.2) (layer "F.Cu") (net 20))
 (segment (start 151.45 60.45) (end 157.95 60.45) (width 0.2) (layer "F.Cu") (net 20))
 (segment (start 151.75 48.97) (end 151.55 48.77) (width 0.2) (layer "F.Cu") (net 20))
 (segment (start 151.45 60.45) (end 151.45 48.87) (width 0.2) (layer "F.Cu") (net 20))
 (segment (start 152.75 47.43) (end 151.55 46.23) (width 0.2) (layer "F.Cu") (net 22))
 (segment (start 143.15 75.85) (end 155.5 75.85) (width 0.2) (layer "F.Cu") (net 22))
 (segment (start 160.65 59.8) (end 152.75 51.9) (width 0.2) (layer "F.Cu") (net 22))
 (segment (start 131.15 87.85) (end 143.15 75.85) (width 0.2) (layer "F.Cu") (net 22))
 (segment (start 130.15 87.85) (end 131.15 87.85) (width 0.2) (layer "F.Cu") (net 22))
 (segment (start 155.5 75.85) (end 160.65 70.7) (width 0.2) (layer "F.Cu") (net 22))
 (segment (start 160.65 70.7) (end 160.65 59.9) (width 0.2) (layer "F.Cu") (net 22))
 (segment (start 152.75 51.9) (end 152.75 47.43) (width 0.2) (layer "F.Cu") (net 22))
 (segment (start 133.4 87.85) (end 133.4 86.5) (width 0.2) (layer "F.Cu") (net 17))
 (segment (start 156.4 76.55) (end 161.95 71) (width 0.2) (layer "F.Cu") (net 17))
 (segment (start 133.4 86.5) (end 143.35 76.55) (width 0.2) (layer "F.Cu") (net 17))
 (segment (start 161.95 71) (end 162 71) (width 0.2) (layer "F.Cu") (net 17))
 (segment (start 162 71) (end 162 60.1) (width 0.2) (layer "F.Cu") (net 17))
 (segment (start 154.09 52.19) (end 154.09 48.77) (width 0.2) (layer "F.Cu") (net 17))
 (segment (start 143.35 76.55) (end 156.4 76.55) (width 0.2) (layer "F.Cu") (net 17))
 (segment (start 162 60.1) (end 154.09 52.19) (width 0.2) (layer "F.Cu") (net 17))
 (segment (start 146.8 90.79) (end 146.8 86.25) (width 0.5) (layer "F.Cu") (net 1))
 (segment (start 108.37 46.23) (end 110.91 46.23) (width 0.2) (layer "F.Cu") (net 1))
 (segment (start 146.8 86.25) (end 147.475 85.575) (width 0.5) (layer "F.Cu") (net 1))
 (segment (start 147.475 85.575) (end 147.475 82.175) (width 0.5) (layer "F.Cu") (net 1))
 (segment (start 130.13 90.97) (end 130.15 90.95) (width 0.2) (layer "F.Cu") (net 23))
 (segment (start 130.13 94.475) (end 130.13 90.97) (width 0.2) (layer "F.Cu") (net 23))
 (segment (start 126.87 94.475) (end 126.87 90.97) (width 0.2) (layer "F.Cu") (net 19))
 (segment (start 126.87 90.97) (end 126.85 90.95) (width 0.2) (layer "F.Cu") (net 19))
 (segment (start 123.4 94.45) (end 123.35 94.5) (width 0.2) (layer "F.Cu") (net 7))
 (segment (start 123.4 90.975) (end 123.4 94.45) (width 0.2) (layer "F.Cu") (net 7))
 (segment (start 133.35 94.475) (end 133.35 91) (width 0.2) (layer "F.Cu") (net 18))
 (segment (start 133.35 91) (end 133.4 90.95) (width 0.2) (layer "F.Cu") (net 18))
 (segment (start 143.73 93.5) (end 156.87 93.5) (width 0.2) (layer "F.Cu") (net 5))
 (segment (start 114.025 76.775) (end 122.75 85.5) (width 0.5) (layer "B.Cu") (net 10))
 (segment (start 146.69 85.5) (end 150.015 82.175) (width 0.5) (layer "B.Cu") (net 10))
 (segment (start 114.025 58.94) (end 114.025 76.775) (width 0.5) (layer "B.Cu") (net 10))
 (segment (start 122.75 85.5) (end 146.69 85.5) (width 0.5) (layer "B.Cu") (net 10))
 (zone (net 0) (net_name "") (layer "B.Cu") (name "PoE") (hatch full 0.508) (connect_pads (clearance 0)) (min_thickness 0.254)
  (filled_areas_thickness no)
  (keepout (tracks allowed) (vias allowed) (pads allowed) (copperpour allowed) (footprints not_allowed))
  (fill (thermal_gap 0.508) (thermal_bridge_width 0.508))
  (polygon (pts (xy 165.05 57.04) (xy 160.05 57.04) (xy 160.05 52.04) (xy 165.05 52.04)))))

